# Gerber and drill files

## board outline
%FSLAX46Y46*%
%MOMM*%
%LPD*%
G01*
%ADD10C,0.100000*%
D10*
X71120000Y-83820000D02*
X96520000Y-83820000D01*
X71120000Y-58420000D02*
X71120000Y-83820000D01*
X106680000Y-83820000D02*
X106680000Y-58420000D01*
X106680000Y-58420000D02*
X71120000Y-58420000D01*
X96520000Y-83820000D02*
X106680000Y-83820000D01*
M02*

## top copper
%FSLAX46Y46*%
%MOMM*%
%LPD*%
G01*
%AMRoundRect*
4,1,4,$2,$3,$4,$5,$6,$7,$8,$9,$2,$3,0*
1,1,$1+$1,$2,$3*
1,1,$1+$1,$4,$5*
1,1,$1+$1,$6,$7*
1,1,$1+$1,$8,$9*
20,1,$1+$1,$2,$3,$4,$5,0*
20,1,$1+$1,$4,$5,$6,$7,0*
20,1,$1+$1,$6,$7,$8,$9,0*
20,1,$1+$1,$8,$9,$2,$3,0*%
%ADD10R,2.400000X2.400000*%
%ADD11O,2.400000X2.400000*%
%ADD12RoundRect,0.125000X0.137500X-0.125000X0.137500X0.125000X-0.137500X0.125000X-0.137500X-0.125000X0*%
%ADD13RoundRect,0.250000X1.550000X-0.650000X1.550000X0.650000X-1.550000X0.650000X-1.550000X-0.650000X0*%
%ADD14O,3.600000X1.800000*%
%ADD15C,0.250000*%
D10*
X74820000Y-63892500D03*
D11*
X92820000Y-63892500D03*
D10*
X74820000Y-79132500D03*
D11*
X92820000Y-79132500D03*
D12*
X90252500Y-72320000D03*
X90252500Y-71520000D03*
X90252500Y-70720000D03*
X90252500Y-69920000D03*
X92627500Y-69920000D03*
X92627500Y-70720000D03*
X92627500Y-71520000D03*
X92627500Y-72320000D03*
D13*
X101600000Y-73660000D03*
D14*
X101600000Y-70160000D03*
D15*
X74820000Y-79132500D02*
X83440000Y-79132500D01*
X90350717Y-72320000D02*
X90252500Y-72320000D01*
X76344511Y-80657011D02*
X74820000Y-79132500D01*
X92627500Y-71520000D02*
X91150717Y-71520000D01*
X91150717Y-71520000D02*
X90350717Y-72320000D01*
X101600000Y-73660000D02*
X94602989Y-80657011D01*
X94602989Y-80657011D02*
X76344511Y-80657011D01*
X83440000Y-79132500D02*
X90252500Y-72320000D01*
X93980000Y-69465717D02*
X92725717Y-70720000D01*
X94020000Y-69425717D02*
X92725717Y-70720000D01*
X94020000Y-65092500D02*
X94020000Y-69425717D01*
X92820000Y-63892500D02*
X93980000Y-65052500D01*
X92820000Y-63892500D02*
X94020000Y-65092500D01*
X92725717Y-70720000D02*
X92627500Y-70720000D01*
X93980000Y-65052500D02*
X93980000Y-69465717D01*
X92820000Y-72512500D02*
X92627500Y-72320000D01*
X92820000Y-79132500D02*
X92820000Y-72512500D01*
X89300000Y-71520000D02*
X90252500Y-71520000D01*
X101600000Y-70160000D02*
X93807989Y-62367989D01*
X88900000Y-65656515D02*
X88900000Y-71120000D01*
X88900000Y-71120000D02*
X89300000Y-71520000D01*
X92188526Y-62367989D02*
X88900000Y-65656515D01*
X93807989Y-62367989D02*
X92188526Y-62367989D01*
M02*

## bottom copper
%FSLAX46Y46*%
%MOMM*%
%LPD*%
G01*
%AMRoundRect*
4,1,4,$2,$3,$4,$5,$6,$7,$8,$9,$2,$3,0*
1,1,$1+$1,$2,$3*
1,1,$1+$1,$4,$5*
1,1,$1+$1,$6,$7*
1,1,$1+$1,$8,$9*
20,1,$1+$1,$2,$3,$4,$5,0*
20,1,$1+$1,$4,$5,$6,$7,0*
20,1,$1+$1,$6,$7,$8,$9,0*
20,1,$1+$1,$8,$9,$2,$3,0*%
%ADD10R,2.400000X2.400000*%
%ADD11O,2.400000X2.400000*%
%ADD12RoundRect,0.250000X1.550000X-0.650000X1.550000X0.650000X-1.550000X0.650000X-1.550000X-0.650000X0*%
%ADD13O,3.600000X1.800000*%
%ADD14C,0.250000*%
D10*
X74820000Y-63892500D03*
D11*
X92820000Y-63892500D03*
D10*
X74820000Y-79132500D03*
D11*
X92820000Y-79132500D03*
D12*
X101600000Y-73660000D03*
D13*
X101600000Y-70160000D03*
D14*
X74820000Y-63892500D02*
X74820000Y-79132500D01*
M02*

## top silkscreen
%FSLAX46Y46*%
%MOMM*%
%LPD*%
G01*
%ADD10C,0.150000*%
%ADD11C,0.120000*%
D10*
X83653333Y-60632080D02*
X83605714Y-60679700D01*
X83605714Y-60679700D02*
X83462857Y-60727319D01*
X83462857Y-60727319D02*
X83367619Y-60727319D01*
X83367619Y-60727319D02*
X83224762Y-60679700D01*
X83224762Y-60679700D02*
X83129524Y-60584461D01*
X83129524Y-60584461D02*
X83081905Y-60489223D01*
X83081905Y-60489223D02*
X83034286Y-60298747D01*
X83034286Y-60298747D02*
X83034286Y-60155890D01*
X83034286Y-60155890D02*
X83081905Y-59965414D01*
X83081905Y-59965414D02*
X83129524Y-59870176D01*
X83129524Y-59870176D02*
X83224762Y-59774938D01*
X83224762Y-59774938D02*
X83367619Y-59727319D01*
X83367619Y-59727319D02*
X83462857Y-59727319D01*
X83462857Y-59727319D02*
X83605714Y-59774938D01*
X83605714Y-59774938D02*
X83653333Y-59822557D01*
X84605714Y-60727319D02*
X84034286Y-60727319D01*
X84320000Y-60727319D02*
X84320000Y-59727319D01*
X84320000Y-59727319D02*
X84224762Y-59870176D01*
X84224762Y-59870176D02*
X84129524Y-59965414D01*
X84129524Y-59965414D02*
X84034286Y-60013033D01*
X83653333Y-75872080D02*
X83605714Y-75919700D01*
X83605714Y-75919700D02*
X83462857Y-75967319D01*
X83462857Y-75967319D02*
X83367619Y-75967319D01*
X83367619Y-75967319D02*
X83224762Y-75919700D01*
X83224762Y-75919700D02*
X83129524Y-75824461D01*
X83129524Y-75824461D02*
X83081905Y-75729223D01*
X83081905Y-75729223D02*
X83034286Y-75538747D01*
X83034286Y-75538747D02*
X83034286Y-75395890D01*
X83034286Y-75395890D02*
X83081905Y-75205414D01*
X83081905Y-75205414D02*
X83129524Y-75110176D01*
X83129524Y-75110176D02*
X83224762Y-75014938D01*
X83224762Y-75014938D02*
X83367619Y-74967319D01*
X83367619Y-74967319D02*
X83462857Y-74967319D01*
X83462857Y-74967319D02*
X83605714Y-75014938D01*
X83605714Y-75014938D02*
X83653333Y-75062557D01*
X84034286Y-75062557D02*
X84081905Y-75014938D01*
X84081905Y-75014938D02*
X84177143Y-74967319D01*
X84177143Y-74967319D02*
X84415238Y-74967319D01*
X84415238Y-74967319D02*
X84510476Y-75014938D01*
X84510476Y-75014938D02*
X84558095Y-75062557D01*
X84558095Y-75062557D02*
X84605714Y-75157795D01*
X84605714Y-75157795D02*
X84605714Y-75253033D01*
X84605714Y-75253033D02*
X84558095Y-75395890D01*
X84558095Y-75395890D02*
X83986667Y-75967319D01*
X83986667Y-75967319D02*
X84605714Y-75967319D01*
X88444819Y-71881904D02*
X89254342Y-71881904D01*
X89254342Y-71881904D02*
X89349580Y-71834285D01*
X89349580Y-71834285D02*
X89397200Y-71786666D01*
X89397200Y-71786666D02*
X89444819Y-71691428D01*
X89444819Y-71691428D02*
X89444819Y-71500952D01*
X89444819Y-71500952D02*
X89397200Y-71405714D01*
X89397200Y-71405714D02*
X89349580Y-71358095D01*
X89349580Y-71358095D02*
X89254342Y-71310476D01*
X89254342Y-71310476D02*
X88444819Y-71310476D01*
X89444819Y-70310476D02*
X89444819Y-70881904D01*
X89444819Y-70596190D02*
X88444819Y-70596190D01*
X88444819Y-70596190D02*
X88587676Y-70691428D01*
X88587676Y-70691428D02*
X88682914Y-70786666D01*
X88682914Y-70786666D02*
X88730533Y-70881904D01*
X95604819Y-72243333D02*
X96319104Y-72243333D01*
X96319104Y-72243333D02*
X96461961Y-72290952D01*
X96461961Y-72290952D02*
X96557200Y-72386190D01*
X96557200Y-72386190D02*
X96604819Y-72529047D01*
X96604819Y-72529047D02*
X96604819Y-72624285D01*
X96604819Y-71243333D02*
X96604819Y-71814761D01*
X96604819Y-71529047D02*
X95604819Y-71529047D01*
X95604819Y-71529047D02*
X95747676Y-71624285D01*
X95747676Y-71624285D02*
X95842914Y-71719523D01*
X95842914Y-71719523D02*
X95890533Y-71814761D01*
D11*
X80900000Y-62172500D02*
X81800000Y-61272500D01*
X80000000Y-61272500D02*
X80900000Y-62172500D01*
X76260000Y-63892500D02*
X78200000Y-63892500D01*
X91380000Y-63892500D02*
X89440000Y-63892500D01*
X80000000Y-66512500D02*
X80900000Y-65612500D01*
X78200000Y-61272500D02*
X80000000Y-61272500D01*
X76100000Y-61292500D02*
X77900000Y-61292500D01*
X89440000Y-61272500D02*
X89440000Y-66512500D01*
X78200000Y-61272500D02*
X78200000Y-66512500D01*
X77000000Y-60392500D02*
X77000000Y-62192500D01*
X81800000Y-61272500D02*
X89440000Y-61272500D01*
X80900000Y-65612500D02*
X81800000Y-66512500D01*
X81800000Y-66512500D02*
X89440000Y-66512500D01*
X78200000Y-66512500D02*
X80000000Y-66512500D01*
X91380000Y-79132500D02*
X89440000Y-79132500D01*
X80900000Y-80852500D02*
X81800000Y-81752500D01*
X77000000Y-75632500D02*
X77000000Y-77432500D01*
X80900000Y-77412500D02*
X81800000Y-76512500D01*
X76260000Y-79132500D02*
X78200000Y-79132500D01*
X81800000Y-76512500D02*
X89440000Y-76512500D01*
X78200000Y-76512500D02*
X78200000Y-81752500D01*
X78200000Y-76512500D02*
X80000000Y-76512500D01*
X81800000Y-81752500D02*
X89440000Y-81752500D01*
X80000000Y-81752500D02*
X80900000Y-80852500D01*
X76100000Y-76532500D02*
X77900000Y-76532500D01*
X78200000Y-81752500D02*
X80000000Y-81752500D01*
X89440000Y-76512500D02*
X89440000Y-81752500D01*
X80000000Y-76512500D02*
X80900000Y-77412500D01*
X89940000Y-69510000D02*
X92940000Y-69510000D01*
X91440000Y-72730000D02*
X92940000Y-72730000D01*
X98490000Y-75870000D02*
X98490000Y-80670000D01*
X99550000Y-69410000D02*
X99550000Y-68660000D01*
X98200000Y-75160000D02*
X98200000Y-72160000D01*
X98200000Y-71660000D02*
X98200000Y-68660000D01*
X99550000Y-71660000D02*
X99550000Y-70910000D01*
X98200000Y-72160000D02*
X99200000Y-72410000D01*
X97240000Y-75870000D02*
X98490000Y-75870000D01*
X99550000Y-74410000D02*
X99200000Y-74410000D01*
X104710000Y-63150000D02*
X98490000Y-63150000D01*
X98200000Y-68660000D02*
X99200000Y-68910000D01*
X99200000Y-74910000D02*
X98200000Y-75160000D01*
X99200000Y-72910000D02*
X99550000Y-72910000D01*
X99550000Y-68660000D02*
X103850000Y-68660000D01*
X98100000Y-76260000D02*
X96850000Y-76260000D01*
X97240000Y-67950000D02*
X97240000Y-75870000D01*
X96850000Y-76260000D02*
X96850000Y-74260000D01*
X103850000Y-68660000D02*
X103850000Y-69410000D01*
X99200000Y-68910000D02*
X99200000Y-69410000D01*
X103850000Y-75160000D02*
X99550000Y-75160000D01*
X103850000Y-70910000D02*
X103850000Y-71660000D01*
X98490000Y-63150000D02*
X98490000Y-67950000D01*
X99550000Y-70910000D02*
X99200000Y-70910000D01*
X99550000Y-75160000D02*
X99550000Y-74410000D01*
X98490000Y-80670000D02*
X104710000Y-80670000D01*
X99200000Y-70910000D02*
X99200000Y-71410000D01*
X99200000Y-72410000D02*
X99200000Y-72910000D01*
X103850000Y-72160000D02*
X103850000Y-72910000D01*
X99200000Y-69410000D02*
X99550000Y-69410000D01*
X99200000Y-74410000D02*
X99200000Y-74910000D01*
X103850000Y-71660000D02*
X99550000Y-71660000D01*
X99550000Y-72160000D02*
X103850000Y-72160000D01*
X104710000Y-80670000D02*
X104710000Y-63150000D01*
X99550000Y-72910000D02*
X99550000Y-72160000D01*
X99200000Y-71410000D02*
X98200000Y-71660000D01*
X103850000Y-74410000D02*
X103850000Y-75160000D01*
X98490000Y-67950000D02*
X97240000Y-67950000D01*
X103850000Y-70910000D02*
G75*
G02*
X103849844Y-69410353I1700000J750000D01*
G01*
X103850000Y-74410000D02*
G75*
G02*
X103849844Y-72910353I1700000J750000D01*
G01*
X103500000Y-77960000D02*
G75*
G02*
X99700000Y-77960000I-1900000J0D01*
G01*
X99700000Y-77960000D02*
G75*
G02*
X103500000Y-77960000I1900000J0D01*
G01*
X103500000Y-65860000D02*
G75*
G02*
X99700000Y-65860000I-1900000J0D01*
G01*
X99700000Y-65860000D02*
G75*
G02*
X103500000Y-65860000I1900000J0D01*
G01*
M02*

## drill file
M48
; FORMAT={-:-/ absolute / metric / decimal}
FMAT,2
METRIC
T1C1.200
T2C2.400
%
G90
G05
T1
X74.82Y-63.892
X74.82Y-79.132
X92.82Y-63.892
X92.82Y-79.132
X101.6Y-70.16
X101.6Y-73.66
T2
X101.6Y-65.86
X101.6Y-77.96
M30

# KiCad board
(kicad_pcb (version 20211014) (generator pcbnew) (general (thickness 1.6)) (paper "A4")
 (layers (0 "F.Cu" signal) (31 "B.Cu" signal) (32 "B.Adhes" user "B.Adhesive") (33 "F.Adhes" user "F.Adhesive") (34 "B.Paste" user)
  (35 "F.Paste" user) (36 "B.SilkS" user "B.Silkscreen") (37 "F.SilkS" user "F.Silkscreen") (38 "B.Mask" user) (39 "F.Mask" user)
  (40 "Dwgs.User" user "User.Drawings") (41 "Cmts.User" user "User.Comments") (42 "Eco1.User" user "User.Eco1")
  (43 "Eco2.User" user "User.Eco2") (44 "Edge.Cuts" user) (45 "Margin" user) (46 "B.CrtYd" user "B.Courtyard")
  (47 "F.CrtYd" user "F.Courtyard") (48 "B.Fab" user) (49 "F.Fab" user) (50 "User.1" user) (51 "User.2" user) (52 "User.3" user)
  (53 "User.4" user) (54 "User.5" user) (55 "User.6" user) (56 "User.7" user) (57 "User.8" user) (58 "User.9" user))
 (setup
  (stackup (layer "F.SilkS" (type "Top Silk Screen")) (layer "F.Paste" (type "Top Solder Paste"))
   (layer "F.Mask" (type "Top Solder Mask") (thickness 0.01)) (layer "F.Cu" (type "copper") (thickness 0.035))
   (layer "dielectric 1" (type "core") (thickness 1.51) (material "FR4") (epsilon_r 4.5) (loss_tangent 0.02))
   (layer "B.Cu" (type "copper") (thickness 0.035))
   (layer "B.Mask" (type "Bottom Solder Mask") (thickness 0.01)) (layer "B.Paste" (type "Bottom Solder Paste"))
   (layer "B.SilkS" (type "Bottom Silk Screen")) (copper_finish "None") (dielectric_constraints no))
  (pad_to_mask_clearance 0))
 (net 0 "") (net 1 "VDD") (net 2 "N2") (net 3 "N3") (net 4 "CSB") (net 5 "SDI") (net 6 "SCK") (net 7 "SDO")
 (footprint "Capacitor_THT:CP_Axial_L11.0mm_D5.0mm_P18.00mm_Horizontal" (layer "F.Cu") (at 74.82 63.8925)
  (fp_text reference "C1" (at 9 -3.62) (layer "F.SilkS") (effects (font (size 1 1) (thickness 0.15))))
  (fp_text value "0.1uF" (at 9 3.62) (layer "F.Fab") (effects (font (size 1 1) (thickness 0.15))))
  (fp_line (start 6.08 -1.72) (end 6.98 -2.62) (layer "F.SilkS") (width 0.12))
  (fp_line (start 5.18 -2.62) (end 6.08 -1.72) (layer "F.SilkS") (width 0.12))
  (fp_line (start 1.44 0) (end 3.38 0) (layer "F.SilkS") (width 0.12))
  (fp_line (start 16.56 0) (end 14.62 0) (layer "F.SilkS") (width 0.12))
  (fp_line (start 5.18 2.62) (end 6.08 1.72) (layer "F.SilkS") (width 0.12))
  (fp_line (start 3.38 -2.62) (end 5.18 -2.62) (layer "F.SilkS") (width 0.12))
  (fp_line (start 1.28 -2.6) (end 3.08 -2.6) (layer "F.SilkS") (width 0.12))
  (fp_line (start 14.62 -2.62) (end 14.62 2.62) (layer "F.SilkS") (width 0.12))
  (fp_line (start 3.38 -2.62) (end 3.38 2.62) (layer "F.SilkS") (width 0.12))
  (fp_line (start 2.18 -3.5) (end 2.18 -1.7) (layer "F.SilkS") (width 0.12))
  (fp_line (start 6.98 -2.62) (end 14.62 -2.62) (layer "F.SilkS") (width 0.12))
  (fp_line (start 6.08 1.72) (end 6.98 2.62) (layer "F.SilkS") (width 0.12))
  (fp_line (start 6.98 2.62) (end 14.62 2.62) (layer "F.SilkS") (width 0.12))
  (fp_line (start 3.38 2.62) (end 5.18 2.62) (layer "F.SilkS") (width 0.12))
  (pad "1" thru_hole rect (at 0 0) (size 2.4 2.4) (drill 1.2) (layers *.Cu *.Mask) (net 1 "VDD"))
  (pad "2" thru_hole oval (at 18 0) (size 2.4 2.4) (drill 1.2) (layers *.Cu *.Mask) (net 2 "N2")))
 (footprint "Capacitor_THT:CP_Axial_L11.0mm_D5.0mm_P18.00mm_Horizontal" (layer "F.Cu") (at 74.82 79.1325)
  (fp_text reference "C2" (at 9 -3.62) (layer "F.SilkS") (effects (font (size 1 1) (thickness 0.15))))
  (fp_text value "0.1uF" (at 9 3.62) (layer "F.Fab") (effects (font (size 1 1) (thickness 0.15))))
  (fp_line (start 16.56 0) (end 14.62 0) (layer "F.SilkS") (width 0.12))
  (fp_line (start 6.08 1.72) (end 6.98 2.62) (layer "F.SilkS") (width 0.12))
  (fp_line (start 2.18 -3.5) (end 2.18 -1.7) (layer "F.SilkS") (width 0.12))
  (fp_line (start 6.08 -1.72) (end 6.98 -2.62) (layer "F.SilkS") (width 0.12))
  (fp_line (start 1.44 0) (end 3.38 0) (layer "F.SilkS") (width 0.12))
  (fp_line (start 6.98 -2.62) (end 14.62 -2.62) (layer "F.SilkS") (width 0.12))
  (fp_line (start 3.38 -2.62) (end 3.38 2.62) (layer "F.SilkS") (width 0.12))
  (fp_line (start 3.38 -2.62) (end 5.18 -2.62) (layer "F.SilkS") (width 0.12))
  (fp_line (start 6.98 2.62) (end 14.62 2.62) (layer "F.SilkS") (width 0.12))
  (fp_line (start 5.18 2.62) (end 6.08 1.72) (layer "F.SilkS") (width 0.12))
  (fp_line (start 1.28 -2.6) (end 3.08 -2.6) (layer "F.SilkS") (width 0.12))
  (fp_line (start 3.38 2.62) (end 5.18 2.62) (layer "F.SilkS") (width 0.12))
  (fp_line (start 14.62 -2.62) (end 14.62 2.62) (layer "F.SilkS") (width 0.12))
  (fp_line (start 5.18 -2.62) (end 6.08 -1.72) (layer "F.SilkS") (width 0.12))
  (pad "1" thru_hole rect (at 0 0) (size 2.4 2.4) (drill 1.2) (layers *.Cu *.Mask) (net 1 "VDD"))
  (pad "2" thru_hole oval (at 18 0) (size 2.4 2.4) (drill 1.2) (layers *.Cu *.Mask) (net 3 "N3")))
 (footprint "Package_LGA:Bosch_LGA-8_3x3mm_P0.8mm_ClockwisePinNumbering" (layer "F.Cu") (at 91.44 71.12 90)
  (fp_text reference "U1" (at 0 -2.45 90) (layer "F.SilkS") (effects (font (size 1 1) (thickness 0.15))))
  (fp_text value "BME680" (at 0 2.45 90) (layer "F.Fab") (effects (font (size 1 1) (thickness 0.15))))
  (fp_line (start 1.61 -1.5) (end 1.61 1.5) (layer "F.SilkS") (width 0.12))
  (fp_line (start -1.61 0) (end -1.61 1.5) (layer "F.SilkS") (width 0.12))
  (pad "1" smd roundrect (at -1.2 -1.1875 90) (size 0.5 0.525) (layers "F.Cu" "F.Paste" "F.Mask") (roundrect_rratio 0.25) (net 1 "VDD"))
  (pad "2" smd roundrect (at -0.4 -1.1875 90) (size 0.5 0.525) (layers "F.Cu" "F.Paste" "F.Mask") (roundrect_rratio 0.25) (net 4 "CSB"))
  (pad "3" smd roundrect (at 0.4 -1.1875 90) (size 0.5 0.525) (layers "F.Cu" "F.Paste" "F.Mask") (roundrect_rratio 0.25) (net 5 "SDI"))
  (pad "4" smd roundrect (at 1.2 -1.1875 90) (size 0.5 0.525) (layers "F.Cu" "F.Paste" "F.Mask") (roundrect_rratio 0.25) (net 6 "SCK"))
  (pad "5" smd roundrect (at 1.2 1.1875 90) (size 0.5 0.525) (layers "F.Cu" "F.Paste" "F.Mask") (roundrect_rratio 0.25) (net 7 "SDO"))
  (pad "6" smd roundrect (at 0.4 1.1875 90) (size 0.5 0.525) (layers "F.Cu" "F.Paste" "F.Mask") (roundrect_rratio 0.25) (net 2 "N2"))
  (pad "7" smd roundrect (at -0.4 1.1875 90) (size 0.5 0.525) (layers "F.Cu" "F.Paste" "F.Mask") (roundrect_rratio 0.25) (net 1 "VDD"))
  (pad "8" smd roundrect (at -1.2 1.1875 90) (size 0.5 0.525) (layers "F.Cu" "F.Paste" "F.Mask") (roundrect_rratio 0.25) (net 3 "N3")))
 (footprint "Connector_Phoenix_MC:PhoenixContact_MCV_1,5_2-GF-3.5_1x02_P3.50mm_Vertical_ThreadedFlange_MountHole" (layer "F.Cu")
  (at 101.6 73.66 90)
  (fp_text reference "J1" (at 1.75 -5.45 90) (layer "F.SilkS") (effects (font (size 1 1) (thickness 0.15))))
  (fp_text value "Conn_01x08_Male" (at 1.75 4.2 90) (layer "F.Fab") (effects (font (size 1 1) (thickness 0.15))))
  (fp_line (start -2.21 -3.11) (end -7.01 -3.11) (layer "F.SilkS") (width 0.12))
  (fp_line (start 4.25 -2.05) (end 5 -2.05) (layer "F.SilkS") (width 0.12))
  (fp_line (start -1.5 -3.4) (end 1.5 -3.4) (layer "F.SilkS") (width 0.12))
  (fp_line (start 2 -3.4) (end 5 -3.4) (layer "F.SilkS") (width 0.12))
  (fp_line (start 2 -2.05) (end 2.75 -2.05) (layer "F.SilkS") (width 0.12))
  (fp_line (start 1.5 -3.4) (end 1.25 -2.4) (layer "F.SilkS") (width 0.12))
  (fp_line (start -2.21 -4.36) (end -2.21 -3.11) (layer "F.SilkS") (width 0.12))
  (fp_line (start -0.75 -2.05) (end -0.75 -2.4) (layer "F.SilkS") (width 0.12))
  (fp_line (start 10.51 3.11) (end 10.51 -3.11) (layer "F.SilkS") (width 0.12))
  (fp_line (start 5 -3.4) (end 4.75 -2.4) (layer "F.SilkS") (width 0.12))
  (fp_line (start -1.25 -2.4) (end -1.5 -3.4) (layer "F.SilkS") (width 0.12))
  (fp_line (start 0.75 -2.4) (end 0.75 -2.05) (layer "F.SilkS") (width 0.12))
  (fp_line (start 5 -2.05) (end 5 2.25) (layer "F.SilkS") (width 0.12))
  (fp_line (start -2.6 -3.5) (end -2.6 -4.75) (layer "F.SilkS") (width 0.12))
  (fp_line (start 5.71 -4.36) (end -2.21 -4.36) (layer "F.SilkS") (width 0.12))
  (fp_line (start -2.6 -4.75) (end -0.6 -4.75) (layer "F.SilkS") (width 0.12))
  (fp_line (start 5 2.25) (end 4.25 2.25) (layer "F.SilkS") (width 0.12))
  (fp_line (start 4.75 -2.4) (end 4.25 -2.4) (layer "F.SilkS") (width 0.12))
  (fp_line (start -1.5 2.25) (end -1.5 -2.05) (layer "F.SilkS") (width 0.12))
  (fp_line (start 2.75 2.25) (end 2 2.25) (layer "F.SilkS") (width 0.12))
  (fp_line (start 10.51 -3.11) (end 5.71 -3.11) (layer "F.SilkS") (width 0.12))
  (fp_line (start 2.75 -2.05) (end 2.75 -2.4) (layer "F.SilkS") (width 0.12))
  (fp_line (start -1.5 -2.05) (end -0.75 -2.05) (layer "F.SilkS") (width 0.12))
  (fp_line (start -7.01 -3.11) (end -7.01 3.11) (layer "F.SilkS") (width 0.12))
  (fp_line (start 2.75 -2.4) (end 2.25 -2.4) (layer "F.SilkS") (width 0.12))
  (fp_line (start 1.25 -2.4) (end 0.75 -2.4) (layer "F.SilkS") (width 0.12))
  (fp_line (start 1.5 2.25) (end 0.75 2.25) (layer "F.SilkS") (width 0.12))
  (fp_line (start 4.25 -2.4) (end 4.25 -2.05) (layer "F.SilkS") (width 0.12))
  (fp_line (start -0.75 -2.4) (end -1.25 -2.4) (layer "F.SilkS") (width 0.12))
  (fp_line (start 2 2.25) (end 2 -2.05) (layer "F.SilkS") (width 0.12))
  (fp_line (start 1.5 -2.05) (end 1.5 2.25) (layer "F.SilkS") (width 0.12))
  (fp_line (start -7.01 3.11) (end 10.51 3.11) (layer "F.SilkS") (width 0.12))
  (fp_line (start 0.75 -2.05) (end 1.5 -2.05) (layer "F.SilkS") (width 0.12))
  (fp_line (start 2.25 -2.4) (end 2 -3.4) (layer "F.SilkS") (width 0.12))
  (fp_line (start -0.75 2.25) (end -1.5 2.25) (layer "F.SilkS") (width 0.12))
  (fp_line (start 5.71 -3.11) (end 5.71 -4.36) (layer "F.SilkS") (width 0.12))
  (fp_arc (start 2.75 2.25) (mid 3.499807 2.09191) (end 4.249647 2.249844) (layer "F.SilkS") (width 0.12))
  (fp_arc (start -0.75 2.25) (mid -0.000193 2.09191) (end 0.749647 2.249844) (layer "F.SilkS") (width 0.12))
  (fp_circle (center -4.3 0) (end -2.4 0) (layer "F.SilkS") (width 0.12) (fill none))
  (fp_circle (center 7.8 0) (end 9.7 0) (layer "F.SilkS") (width 0.12) (fill none))
  (pad "" np_thru_hole circle (at 7.8 0 90) (size 2.4 2.4) (drill 2.4) (layers *.Cu *.Mask))
  (pad "" np_thru_hole circle (at -4.3 0 90) (size 2.4 2.4) (drill 2.4) (layers *.Cu *.Mask))
  (pad "1" thru_hole roundrect (at 0 0 90) (size 1.8 3.6) (drill 1.2) (layers *.Cu *.Mask) (roundrect_rratio 0.138889) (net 1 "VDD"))
  (pad "2" thru_hole oval (at 3.5 0 90) (size 1.8 3.6) (drill 1.2) (layers *.Cu *.Mask) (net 4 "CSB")))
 (gr_line (start 71.12 83.82) (end 96.52 83.82) (layer "Edge.Cuts") (width 0.1))
 (gr_line (start 71.12 58.42) (end 71.12 83.82) (layer "Edge.Cuts") (width 0.1))
 (gr_line (start 106.68 83.82) (end 106.68 58.42) (layer "Edge.Cuts") (width 0.1))
 (gr_line (start 106.68 58.42) (end 71.12 58.42) (layer "Edge.Cuts") (width 0.1))
 (gr_line (start 96.52 83.82) (end 106.68 83.82) (layer "Edge.Cuts") (width 0.1))
 (segment (start 74.82 79.1325) (end 83.44 79.1325) (width 0.25) (layer "F.Cu") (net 1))
 (segment (start 90.350717 72.32) (end 90.2525 72.32) (width 0.25) (layer "F.Cu") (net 1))
 (segment (start 76.344511 80.657011) (end 74.82 79.1325) (width 0.25) (layer "F.Cu") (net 1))
 (segment (start 92.6275 71.52) (end 91.150717 71.52) (width 0.25) (layer "F.Cu") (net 1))
 (segment (start 91.150717 71.52) (end 90.350717 72.32) (width 0.25) (layer "F.Cu") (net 1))
 (segment (start 101.6 73.66) (end 94.602989 80.657011) (width 0.25) (layer "F.Cu") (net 1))
 (segment (start 94.602989 80.657011) (end 76.344511 80.657011) (width 0.25) (layer "F.Cu") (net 1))
 (segment (start 83.44 79.1325) (end 90.2525 72.32) (width 0.25) (layer "F.Cu") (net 1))
 (segment (start 74.82 63.8925) (end 74.82 79.1325) (width 0.25) (layer "B.Cu") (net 1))
 (segment (start 93.98 69.465717) (end 92.725717 70.72) (width 0.25) (layer "F.Cu") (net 2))
 (segment (start 94.02 69.425717) (end 92.725717 70.72) (width 0.25) (layer "F.Cu") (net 2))
 (segment (start 94.02 65.0925) (end 94.02 69.425717) (width 0.25) (layer "F.Cu") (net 2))
 (segment (start 92.82 63.8925) (end 93.98 65.0525) (width 0.25) (layer "F.Cu") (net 2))
 (segment (start 92.82 63.8925) (end 94.02 65.0925) (width 0.25) (layer "F.Cu") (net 2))
 (segment (start 92.725717 70.72) (end 92.6275 70.72) (width 0.25) (layer "F.Cu") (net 2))
 (segment (start 93.98 65.0525) (end 93.98 69.465717) (width 0.25) (layer "F.Cu") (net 2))
 (segment (start 92.82 72.5125) (end 92.6275 72.32) (width 0.25) (layer "F.Cu") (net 3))
 (segment (start 92.82 79.1325) (end 92.82 72.5125) (width 0.25) (layer "F.Cu") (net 3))
 (segment (start 89.3 71.52) (end 90.2525 71.52) (width 0.25) (layer "F.Cu") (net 4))
 (segment (start 101.6 70.16) (end 93.807989 62.367989) (width 0.25) (layer "F.Cu") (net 4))
 (segment (start 88.9 65.656515) (end 88.9 71.12) (width 0.25) (layer "F.Cu") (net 4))
 (segment (start 88.9 71.12) (end 89.3 71.52) (width 0.25) (layer "F.Cu") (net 4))
 (segment (start 92.188526 62.367989) (end 88.9 65.656515) (width 0.25) (layer "F.Cu") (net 4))
 (segment (start 93.807989 62.367989) (end 92.188526 62.367989) (width 0.25) (layer "F.Cu") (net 4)))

